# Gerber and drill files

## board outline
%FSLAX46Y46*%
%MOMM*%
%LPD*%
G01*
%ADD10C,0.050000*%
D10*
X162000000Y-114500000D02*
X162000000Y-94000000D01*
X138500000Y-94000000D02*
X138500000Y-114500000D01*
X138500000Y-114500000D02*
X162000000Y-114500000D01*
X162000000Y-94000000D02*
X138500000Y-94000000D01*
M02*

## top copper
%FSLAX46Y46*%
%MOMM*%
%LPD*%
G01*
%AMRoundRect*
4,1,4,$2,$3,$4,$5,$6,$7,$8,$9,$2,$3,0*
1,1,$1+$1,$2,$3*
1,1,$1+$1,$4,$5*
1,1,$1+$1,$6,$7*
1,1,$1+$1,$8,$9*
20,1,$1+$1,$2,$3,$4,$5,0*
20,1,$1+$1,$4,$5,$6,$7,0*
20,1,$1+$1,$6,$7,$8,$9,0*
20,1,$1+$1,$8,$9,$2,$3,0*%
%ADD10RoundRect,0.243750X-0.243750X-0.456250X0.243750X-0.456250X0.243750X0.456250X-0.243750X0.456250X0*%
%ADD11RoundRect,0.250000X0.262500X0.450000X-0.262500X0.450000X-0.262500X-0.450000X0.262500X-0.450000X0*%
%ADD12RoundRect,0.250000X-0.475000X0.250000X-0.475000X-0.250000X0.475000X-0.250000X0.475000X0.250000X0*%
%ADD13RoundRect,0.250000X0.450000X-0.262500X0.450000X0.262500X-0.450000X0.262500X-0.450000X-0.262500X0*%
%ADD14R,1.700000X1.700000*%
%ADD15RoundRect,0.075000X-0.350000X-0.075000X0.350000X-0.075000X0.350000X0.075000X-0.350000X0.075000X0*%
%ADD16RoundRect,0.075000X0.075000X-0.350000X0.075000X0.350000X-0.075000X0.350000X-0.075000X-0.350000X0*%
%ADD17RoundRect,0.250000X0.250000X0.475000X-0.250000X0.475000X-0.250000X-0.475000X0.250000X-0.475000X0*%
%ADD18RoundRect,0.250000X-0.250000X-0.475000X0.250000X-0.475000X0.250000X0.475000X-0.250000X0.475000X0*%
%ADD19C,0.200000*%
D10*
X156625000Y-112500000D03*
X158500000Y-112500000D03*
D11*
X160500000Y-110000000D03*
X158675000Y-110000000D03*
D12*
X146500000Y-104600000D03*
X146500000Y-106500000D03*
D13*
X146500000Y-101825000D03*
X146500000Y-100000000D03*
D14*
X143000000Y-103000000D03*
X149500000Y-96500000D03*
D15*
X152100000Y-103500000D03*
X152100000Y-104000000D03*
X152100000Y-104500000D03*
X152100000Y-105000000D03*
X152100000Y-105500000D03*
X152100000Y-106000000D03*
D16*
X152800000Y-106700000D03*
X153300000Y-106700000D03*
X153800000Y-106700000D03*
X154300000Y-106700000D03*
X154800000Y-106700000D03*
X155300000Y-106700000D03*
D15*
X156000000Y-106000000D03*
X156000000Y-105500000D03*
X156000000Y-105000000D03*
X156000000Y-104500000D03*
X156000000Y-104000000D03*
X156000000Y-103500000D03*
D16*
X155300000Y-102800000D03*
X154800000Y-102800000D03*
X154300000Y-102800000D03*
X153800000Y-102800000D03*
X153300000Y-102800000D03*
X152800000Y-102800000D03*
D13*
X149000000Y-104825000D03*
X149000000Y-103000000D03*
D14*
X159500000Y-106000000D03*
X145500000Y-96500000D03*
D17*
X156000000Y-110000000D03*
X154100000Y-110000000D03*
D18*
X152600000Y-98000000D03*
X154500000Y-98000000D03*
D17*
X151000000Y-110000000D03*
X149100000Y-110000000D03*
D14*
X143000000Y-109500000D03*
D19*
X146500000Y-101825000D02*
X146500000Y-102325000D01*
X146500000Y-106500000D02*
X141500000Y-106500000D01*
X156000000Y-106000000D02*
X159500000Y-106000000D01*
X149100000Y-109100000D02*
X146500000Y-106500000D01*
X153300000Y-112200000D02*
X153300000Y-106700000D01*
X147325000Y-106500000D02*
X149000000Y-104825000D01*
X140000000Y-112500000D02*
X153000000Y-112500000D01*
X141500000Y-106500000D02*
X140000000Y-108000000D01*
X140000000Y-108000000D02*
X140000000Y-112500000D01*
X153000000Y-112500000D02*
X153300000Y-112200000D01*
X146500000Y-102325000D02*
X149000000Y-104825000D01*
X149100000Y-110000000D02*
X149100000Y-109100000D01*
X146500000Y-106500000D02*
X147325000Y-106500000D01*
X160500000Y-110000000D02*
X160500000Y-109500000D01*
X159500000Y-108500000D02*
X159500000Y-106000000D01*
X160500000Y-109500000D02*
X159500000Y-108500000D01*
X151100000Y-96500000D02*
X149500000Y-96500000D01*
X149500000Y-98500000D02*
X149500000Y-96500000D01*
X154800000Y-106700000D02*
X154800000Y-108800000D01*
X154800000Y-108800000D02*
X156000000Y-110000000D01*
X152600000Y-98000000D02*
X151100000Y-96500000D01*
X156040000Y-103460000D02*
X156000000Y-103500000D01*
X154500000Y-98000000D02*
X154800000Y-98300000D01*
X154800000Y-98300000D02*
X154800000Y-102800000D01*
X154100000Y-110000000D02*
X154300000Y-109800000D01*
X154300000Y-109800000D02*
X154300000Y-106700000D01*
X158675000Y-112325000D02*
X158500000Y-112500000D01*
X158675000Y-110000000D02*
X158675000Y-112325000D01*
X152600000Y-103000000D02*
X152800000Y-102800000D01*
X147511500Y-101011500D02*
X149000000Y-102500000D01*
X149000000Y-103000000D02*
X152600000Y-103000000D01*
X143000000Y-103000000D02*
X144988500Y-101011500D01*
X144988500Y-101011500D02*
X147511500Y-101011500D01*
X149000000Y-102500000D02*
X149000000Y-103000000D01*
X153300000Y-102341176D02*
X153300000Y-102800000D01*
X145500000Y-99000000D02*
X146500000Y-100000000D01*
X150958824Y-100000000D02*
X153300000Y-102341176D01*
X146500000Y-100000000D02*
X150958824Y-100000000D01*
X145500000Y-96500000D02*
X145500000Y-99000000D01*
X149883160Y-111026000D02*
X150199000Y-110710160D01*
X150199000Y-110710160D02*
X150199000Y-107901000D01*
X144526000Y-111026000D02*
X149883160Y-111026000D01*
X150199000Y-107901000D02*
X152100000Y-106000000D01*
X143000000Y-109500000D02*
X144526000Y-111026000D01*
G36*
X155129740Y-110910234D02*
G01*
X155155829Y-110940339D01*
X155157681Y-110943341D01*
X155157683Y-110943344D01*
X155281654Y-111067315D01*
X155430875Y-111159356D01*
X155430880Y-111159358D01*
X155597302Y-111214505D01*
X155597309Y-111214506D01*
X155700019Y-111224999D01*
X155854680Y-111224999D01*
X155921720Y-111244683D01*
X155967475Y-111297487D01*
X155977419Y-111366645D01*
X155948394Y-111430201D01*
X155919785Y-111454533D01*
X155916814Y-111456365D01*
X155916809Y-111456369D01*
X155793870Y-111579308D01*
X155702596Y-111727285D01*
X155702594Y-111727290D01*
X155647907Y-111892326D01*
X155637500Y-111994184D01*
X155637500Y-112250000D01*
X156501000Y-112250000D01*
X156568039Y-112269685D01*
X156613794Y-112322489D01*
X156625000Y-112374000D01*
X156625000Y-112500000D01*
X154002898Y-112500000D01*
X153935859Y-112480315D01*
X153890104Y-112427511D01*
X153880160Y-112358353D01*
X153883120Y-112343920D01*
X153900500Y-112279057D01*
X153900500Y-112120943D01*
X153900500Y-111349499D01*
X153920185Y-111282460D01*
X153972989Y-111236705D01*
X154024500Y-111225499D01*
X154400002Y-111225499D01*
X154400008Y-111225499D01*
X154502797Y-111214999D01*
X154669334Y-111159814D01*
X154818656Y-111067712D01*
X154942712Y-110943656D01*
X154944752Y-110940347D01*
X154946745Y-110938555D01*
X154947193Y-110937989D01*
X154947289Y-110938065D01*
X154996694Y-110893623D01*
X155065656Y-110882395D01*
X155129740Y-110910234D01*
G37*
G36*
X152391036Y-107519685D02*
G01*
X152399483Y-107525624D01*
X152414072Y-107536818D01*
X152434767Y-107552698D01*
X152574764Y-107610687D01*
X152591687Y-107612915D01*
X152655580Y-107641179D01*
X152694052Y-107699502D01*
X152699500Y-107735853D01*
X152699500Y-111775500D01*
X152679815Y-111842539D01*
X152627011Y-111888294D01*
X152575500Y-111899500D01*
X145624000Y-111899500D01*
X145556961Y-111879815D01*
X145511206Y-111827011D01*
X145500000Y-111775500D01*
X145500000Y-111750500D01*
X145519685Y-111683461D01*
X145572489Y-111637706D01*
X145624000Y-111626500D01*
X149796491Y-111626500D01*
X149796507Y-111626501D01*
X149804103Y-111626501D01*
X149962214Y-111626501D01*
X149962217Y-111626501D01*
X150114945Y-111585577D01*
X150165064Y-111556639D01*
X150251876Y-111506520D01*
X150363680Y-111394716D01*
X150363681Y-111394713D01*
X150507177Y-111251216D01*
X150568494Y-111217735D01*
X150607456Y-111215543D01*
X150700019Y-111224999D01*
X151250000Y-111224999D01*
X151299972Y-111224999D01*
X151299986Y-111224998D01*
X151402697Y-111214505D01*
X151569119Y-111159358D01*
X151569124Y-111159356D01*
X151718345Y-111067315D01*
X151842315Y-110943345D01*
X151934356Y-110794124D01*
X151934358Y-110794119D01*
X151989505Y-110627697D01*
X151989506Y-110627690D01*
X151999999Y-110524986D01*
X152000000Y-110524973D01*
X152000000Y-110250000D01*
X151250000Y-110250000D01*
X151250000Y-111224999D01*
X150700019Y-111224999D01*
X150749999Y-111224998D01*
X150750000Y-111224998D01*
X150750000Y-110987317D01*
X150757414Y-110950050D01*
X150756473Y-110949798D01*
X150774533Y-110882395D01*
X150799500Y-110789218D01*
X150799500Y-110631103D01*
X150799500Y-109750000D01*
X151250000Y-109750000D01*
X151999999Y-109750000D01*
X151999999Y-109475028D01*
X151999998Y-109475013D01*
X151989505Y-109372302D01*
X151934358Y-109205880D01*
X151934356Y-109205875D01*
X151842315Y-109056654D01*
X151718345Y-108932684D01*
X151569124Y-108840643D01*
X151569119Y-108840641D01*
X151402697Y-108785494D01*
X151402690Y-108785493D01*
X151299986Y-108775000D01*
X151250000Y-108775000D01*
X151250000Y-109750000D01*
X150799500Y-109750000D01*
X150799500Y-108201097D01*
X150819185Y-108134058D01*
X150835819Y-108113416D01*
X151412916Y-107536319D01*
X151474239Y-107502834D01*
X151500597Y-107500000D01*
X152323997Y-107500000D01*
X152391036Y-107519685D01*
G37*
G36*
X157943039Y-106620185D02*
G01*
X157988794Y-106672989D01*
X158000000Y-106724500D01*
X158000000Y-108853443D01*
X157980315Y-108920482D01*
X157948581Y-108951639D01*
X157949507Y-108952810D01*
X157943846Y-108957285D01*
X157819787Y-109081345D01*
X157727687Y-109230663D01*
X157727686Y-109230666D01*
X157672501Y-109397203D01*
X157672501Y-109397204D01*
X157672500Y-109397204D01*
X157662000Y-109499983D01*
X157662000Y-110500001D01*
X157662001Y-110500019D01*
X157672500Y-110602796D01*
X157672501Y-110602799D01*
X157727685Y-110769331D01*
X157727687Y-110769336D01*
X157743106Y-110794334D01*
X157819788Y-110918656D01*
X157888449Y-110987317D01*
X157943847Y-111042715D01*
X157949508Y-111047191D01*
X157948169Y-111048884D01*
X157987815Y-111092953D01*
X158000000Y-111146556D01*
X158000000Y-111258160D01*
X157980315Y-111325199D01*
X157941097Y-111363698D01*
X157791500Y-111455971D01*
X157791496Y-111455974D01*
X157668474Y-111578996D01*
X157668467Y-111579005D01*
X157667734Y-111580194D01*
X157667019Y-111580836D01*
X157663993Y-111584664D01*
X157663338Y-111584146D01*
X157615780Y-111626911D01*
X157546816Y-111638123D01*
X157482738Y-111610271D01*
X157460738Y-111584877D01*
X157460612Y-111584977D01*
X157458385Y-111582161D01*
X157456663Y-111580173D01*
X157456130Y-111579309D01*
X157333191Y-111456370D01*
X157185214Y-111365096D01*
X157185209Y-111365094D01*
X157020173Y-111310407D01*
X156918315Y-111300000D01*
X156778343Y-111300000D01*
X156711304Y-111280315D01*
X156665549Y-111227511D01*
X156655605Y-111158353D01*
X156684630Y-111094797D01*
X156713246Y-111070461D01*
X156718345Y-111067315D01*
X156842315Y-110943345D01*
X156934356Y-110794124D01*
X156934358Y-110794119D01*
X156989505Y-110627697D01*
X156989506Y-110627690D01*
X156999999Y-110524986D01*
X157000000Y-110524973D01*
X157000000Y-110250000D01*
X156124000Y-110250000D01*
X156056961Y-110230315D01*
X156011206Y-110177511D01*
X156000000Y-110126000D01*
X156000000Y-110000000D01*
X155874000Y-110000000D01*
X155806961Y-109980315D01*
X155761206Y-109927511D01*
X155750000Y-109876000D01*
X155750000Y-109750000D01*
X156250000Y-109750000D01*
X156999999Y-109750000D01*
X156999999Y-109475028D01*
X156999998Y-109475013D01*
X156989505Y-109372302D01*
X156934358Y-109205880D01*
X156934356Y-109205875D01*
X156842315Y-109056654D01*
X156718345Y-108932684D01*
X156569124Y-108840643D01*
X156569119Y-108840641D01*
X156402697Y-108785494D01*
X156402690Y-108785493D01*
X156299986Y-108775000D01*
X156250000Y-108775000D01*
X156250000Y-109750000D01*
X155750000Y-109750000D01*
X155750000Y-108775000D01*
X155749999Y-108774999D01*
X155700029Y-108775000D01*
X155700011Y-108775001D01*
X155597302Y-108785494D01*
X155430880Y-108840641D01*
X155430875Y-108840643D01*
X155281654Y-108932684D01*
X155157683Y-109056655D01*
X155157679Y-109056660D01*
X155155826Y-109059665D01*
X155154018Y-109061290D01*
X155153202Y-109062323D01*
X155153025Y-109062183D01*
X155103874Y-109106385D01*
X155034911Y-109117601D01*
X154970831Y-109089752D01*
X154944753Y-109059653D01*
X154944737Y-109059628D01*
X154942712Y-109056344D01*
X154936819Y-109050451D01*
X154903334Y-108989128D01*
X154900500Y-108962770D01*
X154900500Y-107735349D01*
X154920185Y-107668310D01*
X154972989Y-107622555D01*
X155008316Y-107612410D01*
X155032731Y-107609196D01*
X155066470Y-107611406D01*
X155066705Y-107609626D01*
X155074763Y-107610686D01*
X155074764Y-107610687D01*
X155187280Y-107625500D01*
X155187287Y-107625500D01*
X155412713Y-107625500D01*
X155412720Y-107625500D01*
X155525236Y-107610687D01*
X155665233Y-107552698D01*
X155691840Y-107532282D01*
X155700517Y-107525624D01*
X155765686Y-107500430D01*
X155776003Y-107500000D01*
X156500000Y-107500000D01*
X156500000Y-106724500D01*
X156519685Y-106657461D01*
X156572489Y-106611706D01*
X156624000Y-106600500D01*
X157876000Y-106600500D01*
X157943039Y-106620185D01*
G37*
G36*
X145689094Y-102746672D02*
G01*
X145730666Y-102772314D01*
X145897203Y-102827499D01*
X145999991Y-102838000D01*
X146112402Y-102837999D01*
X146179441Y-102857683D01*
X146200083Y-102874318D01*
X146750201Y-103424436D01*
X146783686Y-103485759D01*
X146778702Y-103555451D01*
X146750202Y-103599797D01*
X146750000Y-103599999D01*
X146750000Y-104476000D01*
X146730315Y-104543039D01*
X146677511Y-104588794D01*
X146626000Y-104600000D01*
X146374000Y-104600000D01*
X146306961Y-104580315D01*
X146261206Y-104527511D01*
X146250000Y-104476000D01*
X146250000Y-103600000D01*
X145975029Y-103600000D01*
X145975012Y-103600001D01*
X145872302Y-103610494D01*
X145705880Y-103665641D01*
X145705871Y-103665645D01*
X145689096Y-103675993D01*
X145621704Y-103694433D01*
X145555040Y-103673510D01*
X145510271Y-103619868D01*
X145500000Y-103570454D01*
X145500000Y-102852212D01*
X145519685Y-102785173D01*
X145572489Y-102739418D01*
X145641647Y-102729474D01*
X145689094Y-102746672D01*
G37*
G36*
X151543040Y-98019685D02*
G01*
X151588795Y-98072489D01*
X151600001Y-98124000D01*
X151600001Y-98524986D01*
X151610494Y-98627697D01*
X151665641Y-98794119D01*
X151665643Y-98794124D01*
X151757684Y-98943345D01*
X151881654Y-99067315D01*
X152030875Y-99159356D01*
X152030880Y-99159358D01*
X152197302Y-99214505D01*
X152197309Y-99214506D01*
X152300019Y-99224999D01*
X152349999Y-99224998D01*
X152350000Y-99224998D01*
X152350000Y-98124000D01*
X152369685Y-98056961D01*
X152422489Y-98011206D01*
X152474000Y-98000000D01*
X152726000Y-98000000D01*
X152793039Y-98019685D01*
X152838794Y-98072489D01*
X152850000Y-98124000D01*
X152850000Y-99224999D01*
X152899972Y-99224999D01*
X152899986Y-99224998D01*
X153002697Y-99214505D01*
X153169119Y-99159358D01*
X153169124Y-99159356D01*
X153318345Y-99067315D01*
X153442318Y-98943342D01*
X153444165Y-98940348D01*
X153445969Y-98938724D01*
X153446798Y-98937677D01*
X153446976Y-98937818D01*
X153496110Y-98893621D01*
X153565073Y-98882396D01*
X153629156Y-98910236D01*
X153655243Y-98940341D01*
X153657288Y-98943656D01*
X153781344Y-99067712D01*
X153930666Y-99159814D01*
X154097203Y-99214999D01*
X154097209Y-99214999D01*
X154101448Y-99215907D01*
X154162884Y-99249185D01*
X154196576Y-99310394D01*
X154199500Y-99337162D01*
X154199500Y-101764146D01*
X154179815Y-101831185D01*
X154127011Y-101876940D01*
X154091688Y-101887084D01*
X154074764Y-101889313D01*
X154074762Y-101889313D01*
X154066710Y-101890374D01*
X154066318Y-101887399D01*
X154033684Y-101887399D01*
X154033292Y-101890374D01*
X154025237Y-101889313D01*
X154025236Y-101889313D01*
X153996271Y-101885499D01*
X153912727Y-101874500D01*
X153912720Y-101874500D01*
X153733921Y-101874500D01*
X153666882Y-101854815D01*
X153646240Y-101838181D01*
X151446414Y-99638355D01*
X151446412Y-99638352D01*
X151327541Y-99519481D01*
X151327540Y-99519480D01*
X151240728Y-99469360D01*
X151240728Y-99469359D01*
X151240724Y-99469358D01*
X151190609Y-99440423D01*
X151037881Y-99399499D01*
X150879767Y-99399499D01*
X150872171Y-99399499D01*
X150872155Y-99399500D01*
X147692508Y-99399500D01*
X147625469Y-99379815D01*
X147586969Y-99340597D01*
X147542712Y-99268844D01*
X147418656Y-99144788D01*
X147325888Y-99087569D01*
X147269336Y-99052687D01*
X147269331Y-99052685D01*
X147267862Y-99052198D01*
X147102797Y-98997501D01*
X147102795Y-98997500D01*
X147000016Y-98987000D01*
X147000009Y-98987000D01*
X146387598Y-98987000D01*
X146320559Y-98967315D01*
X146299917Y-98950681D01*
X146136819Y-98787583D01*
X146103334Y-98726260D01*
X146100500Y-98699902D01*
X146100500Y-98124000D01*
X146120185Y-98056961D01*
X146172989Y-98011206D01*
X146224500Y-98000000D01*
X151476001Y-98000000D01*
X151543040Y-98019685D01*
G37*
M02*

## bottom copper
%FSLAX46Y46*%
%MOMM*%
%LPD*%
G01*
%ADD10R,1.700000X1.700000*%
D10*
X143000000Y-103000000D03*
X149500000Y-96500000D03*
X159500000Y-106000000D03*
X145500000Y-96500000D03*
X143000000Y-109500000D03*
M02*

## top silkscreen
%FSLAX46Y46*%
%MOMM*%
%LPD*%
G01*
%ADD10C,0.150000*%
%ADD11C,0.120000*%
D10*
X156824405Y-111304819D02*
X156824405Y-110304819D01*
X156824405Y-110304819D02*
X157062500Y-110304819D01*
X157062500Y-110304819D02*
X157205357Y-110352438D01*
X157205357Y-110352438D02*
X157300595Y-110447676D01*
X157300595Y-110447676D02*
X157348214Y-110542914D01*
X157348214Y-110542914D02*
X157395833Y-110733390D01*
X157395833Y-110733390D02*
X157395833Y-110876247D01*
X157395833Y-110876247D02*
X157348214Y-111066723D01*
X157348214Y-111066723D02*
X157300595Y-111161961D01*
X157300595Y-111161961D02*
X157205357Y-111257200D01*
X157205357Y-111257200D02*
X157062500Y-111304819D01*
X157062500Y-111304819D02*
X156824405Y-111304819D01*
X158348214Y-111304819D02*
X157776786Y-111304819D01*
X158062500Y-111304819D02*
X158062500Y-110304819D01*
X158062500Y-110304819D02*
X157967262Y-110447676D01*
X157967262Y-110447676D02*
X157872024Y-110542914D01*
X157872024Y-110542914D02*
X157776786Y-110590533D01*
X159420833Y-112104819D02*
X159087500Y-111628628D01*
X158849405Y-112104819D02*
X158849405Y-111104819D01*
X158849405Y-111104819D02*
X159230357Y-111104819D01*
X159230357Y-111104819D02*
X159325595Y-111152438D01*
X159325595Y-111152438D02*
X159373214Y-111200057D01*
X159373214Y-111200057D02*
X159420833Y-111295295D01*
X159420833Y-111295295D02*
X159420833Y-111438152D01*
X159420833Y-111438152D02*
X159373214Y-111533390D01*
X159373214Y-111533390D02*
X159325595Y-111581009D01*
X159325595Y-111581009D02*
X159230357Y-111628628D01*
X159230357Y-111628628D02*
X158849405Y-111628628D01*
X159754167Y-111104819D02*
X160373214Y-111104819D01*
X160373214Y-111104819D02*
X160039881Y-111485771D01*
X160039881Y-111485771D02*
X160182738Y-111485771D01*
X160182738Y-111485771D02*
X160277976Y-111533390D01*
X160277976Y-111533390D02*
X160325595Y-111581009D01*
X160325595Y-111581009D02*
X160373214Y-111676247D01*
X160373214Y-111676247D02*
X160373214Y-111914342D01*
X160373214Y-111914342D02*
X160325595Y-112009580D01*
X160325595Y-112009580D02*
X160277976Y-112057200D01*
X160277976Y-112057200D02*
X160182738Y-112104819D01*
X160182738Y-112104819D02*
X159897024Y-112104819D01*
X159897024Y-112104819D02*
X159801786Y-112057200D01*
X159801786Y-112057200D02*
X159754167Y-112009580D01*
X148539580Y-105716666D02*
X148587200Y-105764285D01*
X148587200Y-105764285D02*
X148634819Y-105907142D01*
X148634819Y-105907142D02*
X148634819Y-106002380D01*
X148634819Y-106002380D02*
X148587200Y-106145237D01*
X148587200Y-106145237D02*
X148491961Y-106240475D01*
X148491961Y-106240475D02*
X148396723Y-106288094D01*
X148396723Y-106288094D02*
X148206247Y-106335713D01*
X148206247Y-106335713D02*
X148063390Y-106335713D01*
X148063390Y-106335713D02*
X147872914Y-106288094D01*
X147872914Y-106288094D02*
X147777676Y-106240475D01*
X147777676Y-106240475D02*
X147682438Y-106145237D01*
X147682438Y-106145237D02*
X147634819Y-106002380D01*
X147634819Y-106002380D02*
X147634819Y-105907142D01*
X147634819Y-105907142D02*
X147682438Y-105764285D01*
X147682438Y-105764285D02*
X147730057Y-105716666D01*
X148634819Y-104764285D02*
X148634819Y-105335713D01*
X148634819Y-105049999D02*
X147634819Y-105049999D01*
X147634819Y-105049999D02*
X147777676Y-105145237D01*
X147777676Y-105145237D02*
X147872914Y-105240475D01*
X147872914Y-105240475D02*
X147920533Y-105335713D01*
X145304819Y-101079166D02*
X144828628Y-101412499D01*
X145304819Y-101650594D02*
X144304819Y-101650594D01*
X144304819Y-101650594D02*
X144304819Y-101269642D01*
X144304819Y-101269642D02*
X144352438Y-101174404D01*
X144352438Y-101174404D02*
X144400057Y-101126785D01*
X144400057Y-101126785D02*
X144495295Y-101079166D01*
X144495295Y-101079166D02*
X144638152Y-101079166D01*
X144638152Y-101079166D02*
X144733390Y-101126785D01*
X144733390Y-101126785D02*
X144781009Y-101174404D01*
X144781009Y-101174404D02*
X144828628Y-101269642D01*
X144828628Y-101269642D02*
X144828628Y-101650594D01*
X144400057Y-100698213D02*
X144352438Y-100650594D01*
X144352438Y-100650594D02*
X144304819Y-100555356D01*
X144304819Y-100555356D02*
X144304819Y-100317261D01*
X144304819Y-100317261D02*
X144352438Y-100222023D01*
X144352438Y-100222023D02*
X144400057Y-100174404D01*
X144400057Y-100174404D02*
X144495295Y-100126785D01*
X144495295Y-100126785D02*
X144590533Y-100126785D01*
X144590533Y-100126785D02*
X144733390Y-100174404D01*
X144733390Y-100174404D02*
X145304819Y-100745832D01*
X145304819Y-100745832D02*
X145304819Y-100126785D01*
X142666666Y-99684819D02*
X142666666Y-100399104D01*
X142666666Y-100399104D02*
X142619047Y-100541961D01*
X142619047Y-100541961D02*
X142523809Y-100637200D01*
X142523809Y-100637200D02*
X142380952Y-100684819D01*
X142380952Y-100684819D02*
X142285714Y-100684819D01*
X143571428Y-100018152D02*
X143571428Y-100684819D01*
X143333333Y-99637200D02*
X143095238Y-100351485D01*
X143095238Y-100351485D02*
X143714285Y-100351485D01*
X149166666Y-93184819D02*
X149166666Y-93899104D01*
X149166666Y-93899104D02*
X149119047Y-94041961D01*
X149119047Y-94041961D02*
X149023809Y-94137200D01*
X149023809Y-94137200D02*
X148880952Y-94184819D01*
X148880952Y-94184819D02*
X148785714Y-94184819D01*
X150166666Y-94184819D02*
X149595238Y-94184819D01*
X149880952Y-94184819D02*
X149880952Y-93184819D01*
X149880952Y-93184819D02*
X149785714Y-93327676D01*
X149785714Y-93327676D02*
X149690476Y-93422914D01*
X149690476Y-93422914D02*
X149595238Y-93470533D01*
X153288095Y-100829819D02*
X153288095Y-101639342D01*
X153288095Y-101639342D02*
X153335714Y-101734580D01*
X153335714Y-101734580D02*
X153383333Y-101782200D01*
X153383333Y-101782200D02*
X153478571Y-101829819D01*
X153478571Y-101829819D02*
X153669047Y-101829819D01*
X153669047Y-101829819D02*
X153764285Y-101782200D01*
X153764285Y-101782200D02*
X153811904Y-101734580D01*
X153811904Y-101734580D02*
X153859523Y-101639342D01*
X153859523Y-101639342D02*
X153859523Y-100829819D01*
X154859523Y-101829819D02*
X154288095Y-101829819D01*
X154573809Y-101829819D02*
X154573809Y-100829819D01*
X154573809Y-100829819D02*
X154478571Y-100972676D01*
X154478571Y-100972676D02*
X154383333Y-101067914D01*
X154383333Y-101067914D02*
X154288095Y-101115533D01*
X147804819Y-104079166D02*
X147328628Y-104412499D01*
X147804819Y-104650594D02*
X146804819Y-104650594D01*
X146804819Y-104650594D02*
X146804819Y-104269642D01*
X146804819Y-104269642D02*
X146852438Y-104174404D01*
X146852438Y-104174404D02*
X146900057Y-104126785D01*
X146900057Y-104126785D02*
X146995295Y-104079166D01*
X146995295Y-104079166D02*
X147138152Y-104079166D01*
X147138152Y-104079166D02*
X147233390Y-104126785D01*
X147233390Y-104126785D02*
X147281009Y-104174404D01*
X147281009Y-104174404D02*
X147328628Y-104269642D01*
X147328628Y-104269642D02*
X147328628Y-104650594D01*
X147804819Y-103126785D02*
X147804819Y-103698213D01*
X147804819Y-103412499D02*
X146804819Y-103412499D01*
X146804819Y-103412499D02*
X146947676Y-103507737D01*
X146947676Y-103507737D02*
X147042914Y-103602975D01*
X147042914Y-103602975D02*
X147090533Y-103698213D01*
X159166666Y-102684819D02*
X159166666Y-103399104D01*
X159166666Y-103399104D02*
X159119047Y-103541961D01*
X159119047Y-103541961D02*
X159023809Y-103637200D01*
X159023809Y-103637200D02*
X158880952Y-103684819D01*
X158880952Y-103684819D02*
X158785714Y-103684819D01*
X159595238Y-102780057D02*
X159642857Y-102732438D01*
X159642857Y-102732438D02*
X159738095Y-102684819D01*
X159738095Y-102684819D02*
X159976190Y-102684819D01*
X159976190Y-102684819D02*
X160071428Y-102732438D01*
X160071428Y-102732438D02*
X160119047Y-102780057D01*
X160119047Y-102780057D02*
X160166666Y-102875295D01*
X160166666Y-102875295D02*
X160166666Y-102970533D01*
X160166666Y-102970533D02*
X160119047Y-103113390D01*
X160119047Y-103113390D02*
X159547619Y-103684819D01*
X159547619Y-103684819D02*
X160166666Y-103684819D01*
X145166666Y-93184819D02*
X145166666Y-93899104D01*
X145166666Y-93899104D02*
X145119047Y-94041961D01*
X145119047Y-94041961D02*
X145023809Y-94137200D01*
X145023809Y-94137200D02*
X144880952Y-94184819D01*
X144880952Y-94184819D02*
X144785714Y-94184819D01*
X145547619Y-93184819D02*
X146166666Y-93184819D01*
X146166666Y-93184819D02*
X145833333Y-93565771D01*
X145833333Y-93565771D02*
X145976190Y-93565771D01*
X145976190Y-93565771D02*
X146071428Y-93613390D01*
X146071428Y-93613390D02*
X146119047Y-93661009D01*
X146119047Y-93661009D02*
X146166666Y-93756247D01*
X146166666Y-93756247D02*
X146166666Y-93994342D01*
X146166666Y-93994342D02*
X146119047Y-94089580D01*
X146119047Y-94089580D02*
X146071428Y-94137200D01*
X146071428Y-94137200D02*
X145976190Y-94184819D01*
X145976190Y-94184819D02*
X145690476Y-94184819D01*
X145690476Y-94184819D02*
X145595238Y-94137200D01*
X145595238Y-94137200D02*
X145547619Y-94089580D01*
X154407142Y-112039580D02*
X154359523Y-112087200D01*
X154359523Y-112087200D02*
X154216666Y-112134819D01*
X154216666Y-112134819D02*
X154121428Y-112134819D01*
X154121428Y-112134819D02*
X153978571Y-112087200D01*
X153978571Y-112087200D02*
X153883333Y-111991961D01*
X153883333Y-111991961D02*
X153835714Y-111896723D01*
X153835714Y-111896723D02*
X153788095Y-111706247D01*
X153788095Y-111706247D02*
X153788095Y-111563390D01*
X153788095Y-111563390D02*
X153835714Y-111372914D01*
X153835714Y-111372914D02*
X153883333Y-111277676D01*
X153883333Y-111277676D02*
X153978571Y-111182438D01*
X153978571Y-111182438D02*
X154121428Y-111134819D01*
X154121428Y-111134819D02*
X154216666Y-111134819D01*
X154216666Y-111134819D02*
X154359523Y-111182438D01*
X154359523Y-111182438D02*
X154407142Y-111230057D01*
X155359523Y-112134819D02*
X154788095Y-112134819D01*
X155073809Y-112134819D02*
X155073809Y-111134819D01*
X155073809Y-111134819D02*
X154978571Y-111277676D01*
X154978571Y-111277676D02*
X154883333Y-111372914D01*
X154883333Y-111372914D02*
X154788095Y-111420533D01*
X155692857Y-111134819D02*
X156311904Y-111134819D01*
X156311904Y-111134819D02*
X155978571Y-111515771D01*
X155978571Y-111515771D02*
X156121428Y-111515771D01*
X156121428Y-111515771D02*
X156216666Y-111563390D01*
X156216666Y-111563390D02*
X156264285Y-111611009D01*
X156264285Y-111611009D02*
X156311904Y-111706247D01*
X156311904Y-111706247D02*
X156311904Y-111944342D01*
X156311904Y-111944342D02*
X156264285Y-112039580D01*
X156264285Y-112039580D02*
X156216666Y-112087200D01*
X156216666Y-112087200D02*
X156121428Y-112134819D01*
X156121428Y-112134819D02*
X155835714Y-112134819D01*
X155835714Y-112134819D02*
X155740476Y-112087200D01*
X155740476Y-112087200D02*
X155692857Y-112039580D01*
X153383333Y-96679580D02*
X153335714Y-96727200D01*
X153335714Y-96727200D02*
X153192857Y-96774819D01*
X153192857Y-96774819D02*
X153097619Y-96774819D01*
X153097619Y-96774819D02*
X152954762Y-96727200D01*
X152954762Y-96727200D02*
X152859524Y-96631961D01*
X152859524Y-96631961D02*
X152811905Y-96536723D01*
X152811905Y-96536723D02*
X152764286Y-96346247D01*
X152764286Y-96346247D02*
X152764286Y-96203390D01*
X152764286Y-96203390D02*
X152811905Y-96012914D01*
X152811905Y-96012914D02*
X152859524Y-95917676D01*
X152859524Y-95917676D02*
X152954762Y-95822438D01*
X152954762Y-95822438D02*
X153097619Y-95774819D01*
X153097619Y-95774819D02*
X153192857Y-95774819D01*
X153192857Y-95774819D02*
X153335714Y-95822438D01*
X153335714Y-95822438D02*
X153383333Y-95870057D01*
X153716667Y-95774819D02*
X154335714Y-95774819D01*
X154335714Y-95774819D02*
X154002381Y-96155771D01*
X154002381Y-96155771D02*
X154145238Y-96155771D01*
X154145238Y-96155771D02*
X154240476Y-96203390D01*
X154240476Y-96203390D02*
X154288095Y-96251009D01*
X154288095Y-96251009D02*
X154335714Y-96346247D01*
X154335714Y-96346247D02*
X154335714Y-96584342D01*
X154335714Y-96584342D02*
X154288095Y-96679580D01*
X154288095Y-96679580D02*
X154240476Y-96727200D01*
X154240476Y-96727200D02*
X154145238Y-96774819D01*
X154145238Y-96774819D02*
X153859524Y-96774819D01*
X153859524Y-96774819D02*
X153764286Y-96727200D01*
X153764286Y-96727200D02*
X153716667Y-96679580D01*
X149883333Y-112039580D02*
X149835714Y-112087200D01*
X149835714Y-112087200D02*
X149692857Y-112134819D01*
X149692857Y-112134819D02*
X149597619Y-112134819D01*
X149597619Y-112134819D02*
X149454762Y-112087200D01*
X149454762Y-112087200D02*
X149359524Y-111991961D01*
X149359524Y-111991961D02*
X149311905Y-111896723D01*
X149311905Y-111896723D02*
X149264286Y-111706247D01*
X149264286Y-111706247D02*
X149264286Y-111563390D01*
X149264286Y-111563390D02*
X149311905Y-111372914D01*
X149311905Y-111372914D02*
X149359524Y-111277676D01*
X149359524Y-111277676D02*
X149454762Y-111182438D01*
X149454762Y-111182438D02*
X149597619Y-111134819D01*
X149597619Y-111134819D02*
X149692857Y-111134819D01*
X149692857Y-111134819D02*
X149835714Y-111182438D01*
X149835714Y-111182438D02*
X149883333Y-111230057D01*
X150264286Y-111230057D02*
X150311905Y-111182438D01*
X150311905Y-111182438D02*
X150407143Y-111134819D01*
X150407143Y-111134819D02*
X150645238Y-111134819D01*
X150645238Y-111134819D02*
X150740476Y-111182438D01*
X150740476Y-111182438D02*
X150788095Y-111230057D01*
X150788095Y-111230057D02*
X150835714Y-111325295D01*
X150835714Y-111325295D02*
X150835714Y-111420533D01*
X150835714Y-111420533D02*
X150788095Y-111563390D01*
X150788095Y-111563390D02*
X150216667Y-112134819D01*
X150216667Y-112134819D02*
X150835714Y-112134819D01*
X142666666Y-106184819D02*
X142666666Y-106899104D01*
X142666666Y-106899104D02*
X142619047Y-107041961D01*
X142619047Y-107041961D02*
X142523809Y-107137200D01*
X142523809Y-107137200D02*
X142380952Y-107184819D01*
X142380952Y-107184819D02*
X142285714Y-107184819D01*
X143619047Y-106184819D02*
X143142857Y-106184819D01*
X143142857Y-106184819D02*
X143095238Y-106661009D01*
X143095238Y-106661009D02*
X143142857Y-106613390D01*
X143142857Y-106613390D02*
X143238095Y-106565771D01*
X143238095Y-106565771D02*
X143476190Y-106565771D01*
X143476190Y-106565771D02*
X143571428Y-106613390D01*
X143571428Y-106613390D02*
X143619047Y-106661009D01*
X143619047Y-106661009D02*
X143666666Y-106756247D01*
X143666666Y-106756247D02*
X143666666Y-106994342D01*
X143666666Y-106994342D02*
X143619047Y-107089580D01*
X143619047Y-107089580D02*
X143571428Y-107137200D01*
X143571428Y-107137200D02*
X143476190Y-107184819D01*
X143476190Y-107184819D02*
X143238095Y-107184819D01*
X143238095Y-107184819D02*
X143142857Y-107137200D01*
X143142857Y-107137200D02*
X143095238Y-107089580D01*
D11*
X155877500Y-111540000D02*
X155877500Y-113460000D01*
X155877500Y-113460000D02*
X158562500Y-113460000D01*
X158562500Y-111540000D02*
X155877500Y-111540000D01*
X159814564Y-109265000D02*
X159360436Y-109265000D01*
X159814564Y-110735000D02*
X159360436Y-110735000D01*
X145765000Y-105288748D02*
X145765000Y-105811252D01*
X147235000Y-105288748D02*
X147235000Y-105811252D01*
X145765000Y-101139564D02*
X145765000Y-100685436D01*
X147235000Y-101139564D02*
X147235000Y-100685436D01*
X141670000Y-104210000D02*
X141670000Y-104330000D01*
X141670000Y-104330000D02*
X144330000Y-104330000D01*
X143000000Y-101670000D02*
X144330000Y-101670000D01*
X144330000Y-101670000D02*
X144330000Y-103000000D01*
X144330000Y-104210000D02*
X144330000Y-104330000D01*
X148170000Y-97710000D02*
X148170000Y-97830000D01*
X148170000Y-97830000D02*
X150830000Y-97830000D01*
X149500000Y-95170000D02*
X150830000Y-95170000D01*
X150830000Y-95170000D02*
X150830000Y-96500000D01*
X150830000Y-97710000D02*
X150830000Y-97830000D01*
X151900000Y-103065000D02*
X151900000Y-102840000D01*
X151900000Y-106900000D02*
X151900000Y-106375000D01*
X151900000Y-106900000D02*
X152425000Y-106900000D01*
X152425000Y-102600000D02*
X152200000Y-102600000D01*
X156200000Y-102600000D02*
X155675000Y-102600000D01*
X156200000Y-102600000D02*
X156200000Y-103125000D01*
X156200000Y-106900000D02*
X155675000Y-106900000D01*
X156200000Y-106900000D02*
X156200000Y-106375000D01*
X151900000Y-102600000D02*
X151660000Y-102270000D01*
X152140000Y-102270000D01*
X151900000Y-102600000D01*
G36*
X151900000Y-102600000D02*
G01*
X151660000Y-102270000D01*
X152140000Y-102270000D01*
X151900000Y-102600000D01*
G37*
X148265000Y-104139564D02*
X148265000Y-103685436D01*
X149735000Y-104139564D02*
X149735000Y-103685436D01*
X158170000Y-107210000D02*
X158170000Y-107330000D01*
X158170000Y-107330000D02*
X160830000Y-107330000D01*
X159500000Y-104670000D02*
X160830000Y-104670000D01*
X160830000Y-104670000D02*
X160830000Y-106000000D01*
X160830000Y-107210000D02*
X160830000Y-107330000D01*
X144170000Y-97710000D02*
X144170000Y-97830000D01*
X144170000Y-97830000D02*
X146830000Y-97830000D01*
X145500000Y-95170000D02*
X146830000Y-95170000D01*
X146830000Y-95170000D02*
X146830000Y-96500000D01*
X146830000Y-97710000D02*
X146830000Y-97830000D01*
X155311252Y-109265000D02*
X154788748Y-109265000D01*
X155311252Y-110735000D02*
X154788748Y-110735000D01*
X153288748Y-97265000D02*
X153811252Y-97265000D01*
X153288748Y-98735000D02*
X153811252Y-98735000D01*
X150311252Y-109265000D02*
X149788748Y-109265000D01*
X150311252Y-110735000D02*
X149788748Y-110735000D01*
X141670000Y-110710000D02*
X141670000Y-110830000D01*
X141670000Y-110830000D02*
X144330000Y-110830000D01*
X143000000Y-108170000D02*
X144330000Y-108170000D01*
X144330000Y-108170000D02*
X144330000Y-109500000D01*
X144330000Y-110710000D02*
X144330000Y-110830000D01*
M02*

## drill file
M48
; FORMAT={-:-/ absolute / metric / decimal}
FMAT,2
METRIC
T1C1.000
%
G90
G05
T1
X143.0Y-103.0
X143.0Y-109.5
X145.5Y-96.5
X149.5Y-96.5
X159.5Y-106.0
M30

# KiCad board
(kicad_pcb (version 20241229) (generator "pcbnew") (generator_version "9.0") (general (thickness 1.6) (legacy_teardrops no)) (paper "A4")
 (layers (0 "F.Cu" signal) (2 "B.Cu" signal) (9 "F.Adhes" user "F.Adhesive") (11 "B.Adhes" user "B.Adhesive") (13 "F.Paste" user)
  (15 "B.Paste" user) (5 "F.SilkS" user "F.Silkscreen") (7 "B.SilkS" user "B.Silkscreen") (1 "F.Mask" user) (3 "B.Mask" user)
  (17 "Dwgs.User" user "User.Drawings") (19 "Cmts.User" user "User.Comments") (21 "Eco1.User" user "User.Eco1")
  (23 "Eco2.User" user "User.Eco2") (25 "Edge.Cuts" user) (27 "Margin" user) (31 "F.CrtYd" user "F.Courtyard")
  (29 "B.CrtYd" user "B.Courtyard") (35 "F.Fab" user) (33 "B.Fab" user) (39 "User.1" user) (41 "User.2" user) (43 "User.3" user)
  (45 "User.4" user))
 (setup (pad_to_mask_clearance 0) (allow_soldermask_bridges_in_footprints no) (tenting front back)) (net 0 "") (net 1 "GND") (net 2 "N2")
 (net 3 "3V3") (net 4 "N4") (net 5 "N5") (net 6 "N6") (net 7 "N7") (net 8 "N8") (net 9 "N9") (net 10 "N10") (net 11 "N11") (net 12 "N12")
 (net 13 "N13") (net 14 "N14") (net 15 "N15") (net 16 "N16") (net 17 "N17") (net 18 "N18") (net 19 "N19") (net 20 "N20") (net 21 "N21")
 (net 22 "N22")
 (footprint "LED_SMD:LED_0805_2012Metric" (layer "F.Cu") (at 157.5625 112.5)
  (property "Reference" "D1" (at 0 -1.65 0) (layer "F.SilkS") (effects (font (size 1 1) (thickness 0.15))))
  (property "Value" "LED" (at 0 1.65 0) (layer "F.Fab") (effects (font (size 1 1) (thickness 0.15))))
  (fp_line (start -1.685 -0.96) (end -1.685 0.96) (stroke (width 0.12) (type solid)) (layer "F.SilkS"))
  (fp_line (start -1.685 0.96) (end 1 0.96) (stroke (width 0.12) (type solid)) (layer "F.SilkS"))
  (fp_line (start 1 -0.96) (end -1.685 -0.96) (stroke (width 0.12) (type solid)) (layer "F.SilkS"))
  (pad "1" smd roundrect (at -0.9375 0) (size 0.975 1.4) (layers "F.Cu" "F.Mask" "F.Paste") (roundrect_rratio 0.25) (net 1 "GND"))
  (pad "2" smd roundrect (at 0.9375 0) (size 0.975 1.4) (layers "F.Cu" "F.Mask" "F.Paste") (roundrect_rratio 0.25) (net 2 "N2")))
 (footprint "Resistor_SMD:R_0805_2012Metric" (layer "F.Cu") (at 159.5875 110 180)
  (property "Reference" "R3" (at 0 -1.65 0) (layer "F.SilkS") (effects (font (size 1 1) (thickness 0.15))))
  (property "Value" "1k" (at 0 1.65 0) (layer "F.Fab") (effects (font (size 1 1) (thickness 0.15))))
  (fp_line (start -0.227064 0.735) (end 0.227064 0.735) (stroke (width 0.12) (type solid)) (layer "F.SilkS"))
  (fp_line (start -0.227064 -0.735) (end 0.227064 -0.735) (stroke (width 0.12) (type solid)) (layer "F.SilkS"))
  (pad "1" smd roundrect (at -0.9125 0 180) (size 1.025 1.4) (layers "F.Cu" "F.Mask" "F.Paste") (roundrect_rratio 0.243902) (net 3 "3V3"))
  (pad "2" smd roundrect (at 0.9125 0 180) (size 1.025 1.4) (layers "F.Cu" "F.Mask" "F.Paste") (roundrect_rratio 0.243902) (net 2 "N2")))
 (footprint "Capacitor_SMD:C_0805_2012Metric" (layer "F.Cu") (at 146.5 105.55 -90)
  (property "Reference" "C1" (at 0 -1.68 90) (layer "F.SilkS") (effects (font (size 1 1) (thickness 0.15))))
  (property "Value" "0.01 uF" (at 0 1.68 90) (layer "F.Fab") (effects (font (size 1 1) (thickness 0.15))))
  (fp_line (start -0.261252 0.735) (end 0.261252 0.735) (stroke (width 0.12) (type solid)) (layer "F.SilkS"))
  (fp_line (start -0.261252 -0.735) (end 0.261252 -0.735) (stroke (width 0.12) (type solid)) (layer "F.SilkS"))
  (pad "1" smd roundrect (at -0.95 0 270) (size 1 1.45) (layers "F.Cu" "F.Mask" "F.Paste") (roundrect_rratio 0.25) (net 1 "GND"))
  (pad "2" smd roundrect (at 0.95 0 270) (size 1 1.45) (layers "F.Cu" "F.Mask" "F.Paste") (roundrect_rratio 0.25) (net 3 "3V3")))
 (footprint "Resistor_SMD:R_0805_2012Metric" (layer "F.Cu") (at 146.5 100.9125 90)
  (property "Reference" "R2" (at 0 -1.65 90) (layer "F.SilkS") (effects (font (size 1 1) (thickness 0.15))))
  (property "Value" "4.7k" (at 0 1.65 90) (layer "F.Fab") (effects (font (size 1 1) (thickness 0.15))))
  (fp_line (start -0.227064 -0.735) (end 0.227064 -0.735) (stroke (width 0.12) (type solid)) (layer "F.SilkS"))
  (fp_line (start -0.227064 0.735) (end 0.227064 0.735) (stroke (width 0.12) (type solid)) (layer "F.SilkS"))
  (pad "1" smd roundrect (at -0.9125 0 90) (size 1.025 1.4) (layers "F.Cu" "F.Mask" "F.Paste") (roundrect_rratio 0.243902) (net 3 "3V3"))
  (pad "2" smd roundrect (at 0.9125 0 90) (size 1.025 1.4) (layers "F.Cu" "F.Mask" "F.Paste") (roundrect_rratio 0.243902) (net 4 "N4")))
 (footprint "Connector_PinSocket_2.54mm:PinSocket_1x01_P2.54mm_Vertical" (layer "F.Cu") (at 143 103)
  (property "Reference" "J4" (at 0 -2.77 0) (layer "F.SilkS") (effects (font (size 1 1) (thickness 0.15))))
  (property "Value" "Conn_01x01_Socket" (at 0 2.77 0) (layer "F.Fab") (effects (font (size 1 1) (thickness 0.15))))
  (fp_line (start -1.33 1.21) (end -1.33 1.33) (stroke (width 0.12) (type solid)) (layer "F.SilkS"))
  (fp_line (start -1.33 1.33) (end 1.33 1.33) (stroke (width 0.12) (type solid)) (layer "F.SilkS"))
  (fp_line (start 0 -1.33) (end 1.33 -1.33) (stroke (width 0.12) (type solid)) (layer "F.SilkS"))
  (fp_line (start 1.33 -1.33) (end 1.33 0) (stroke (width 0.12) (type solid)) (layer "F.SilkS"))
  (fp_line (start 1.33 1.21) (end 1.33 1.33) (stroke (width 0.12) (type solid)) (layer "F.SilkS"))
  (pad "1" thru_hole rect (at 0 0) (size 1.7 1.7) (drill 1) (layers "*.Cu" "*.Mask") (remove_unused_layers no) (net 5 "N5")))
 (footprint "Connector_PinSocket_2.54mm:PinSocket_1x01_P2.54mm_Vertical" (layer "F.Cu") (at 149.5 96.5)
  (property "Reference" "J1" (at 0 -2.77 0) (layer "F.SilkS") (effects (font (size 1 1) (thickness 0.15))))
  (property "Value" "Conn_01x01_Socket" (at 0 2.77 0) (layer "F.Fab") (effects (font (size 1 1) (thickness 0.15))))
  (fp_line (start -1.33 1.21) (end -1.33 1.33) (stroke (width 0.12) (type solid)) (layer "F.SilkS"))
  (fp_line (start -1.33 1.33) (end 1.33 1.33) (stroke (width 0.12) (type solid)) (layer "F.SilkS"))
  (fp_line (start 0 -1.33) (end 1.33 -1.33) (stroke (width 0.12) (type solid)) (layer "F.SilkS"))
  (fp_line (start 1.33 -1.33) (end 1.33 0) (stroke (width 0.12) (type solid)) (layer "F.SilkS"))
  (fp_line (start 1.33 1.21) (end 1.33 1.33) (stroke (width 0.12) (type solid)) (layer "F.SilkS"))
  (pad "1" thru_hole rect (at 0 0) (size 1.7 1.7) (drill 1) (layers "*.Cu" "*.Mask") (remove_unused_layers no) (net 1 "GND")))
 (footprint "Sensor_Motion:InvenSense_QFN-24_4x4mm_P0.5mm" (layer "F.Cu") (at 154.05 104.75)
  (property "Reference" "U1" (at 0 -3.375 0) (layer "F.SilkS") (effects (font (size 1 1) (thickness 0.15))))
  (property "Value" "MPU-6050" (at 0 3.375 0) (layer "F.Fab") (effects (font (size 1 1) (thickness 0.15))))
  (fp_line (start -2.15 -1.685) (end -2.15 -1.91) (stroke (width 0.12) (type solid)) (layer "F.SilkS"))
  (fp_line (start -2.15 2.15) (end -2.15 1.625) (stroke (width 0.12) (type solid)) (layer "F.SilkS"))
  (fp_line (start -2.15 2.15) (end -1.625 2.15) (stroke (width 0.12) (type solid)) (layer "F.SilkS"))
  (fp_line (start -1.625 -2.15) (end -1.85 -2.15) (stroke (width 0.12) (type solid)) (layer "F.SilkS"))
  (fp_line (start 2.15 -2.15) (end 1.625 -2.15) (stroke (width 0.12) (type solid)) (layer "F.SilkS"))
  (fp_line (start 2.15 -2.15) (end 2.15 -1.625) (stroke (width 0.12) (type solid)) (layer "F.SilkS"))
  (fp_line (start 2.15 2.15) (end 1.625 2.15) (stroke (width 0.12) (type solid)) (layer "F.SilkS"))
  (fp_line (start 2.15 2.15) (end 2.15 1.625) (stroke (width 0.12) (type solid)) (layer "F.SilkS"))
  (fp_poly
   (pts (xy -2.15 -2.15) (xy -2.39 -2.48) (xy -1.91 -2.48) (xy -2.15 -2.15)) (stroke (width 0.12) (type solid)) (fill yes) (layer "F.SilkS"))
  (pad "1" smd roundrect (at -1.95 -1.25) (size 0.85 0.3) (layers "F.Cu" "F.Mask" "F.Paste") (roundrect_rratio 0.25) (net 1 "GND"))
  (pad "2" smd roundrect (at -1.95 -0.75) (size 0.85 0.3) (layers "F.Cu" "F.Mask" "F.Paste") (roundrect_rratio 0.25) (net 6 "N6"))
  (pad "3" smd roundrect (at -1.95 -0.25) (size 0.85 0.3) (layers "F.Cu" "F.Mask" "F.Paste") (roundrect_rratio 0.25) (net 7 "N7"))
  (pad "4" smd roundrect (at -1.95 0.25) (size 0.85 0.3) (layers "F.Cu" "F.Mask" "F.Paste") (roundrect_rratio 0.25) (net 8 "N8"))
  (pad "5" smd roundrect (at -1.95 0.75) (size 0.85 0.3) (layers "F.Cu" "F.Mask" "F.Paste") (roundrect_rratio 0.25) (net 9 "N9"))
  (pad "6" smd roundrect (at -1.95 1.25) (size 0.85 0.3) (layers "F.Cu" "F.Mask" "F.Paste") (roundrect_rratio 0.25) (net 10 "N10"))
  (pad "7" smd roundrect (at -1.25 1.95 90) (size 0.85 0.3) (layers "F.Cu" "F.Mask" "F.Paste") (roundrect_rratio 0.25) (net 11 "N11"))
  (pad "8" smd roundrect (at -0.75 1.95 90) (size 0.85 0.3) (layers "F.Cu" "F.Mask" "F.Paste") (roundrect_rratio 0.25) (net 3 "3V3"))
  (pad "9" smd roundrect (at -0.25 1.95 90) (size 0.85 0.3) (layers "F.Cu" "F.Mask" "F.Paste") (roundrect_rratio 0.25) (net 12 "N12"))
  (pad "10" smd roundrect (at 0.25 1.95 90) (size 0.85 0.3) (layers "F.Cu" "F.Mask" "F.Paste") (roundrect_rratio 0.25) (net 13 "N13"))
  (pad "11" smd roundrect (at 0.75 1.95 90) (size 0.85 0.3) (layers "F.Cu" "F.Mask" "F.Paste") (roundrect_rratio 0.25) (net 1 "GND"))
  (pad "12" smd roundrect (at 1.25 1.95 90) (size 0.85 0.3) (layers "F.Cu" "F.Mask" "F.Paste") (roundrect_rratio 0.25) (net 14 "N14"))
  (pad "13" smd roundrect (at 1.95 1.25) (size 0.85 0.3) (layers "F.Cu" "F.Mask" "F.Paste") (roundrect_rratio 0.25) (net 3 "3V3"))
  (pad "14" smd roundrect (at 1.95 0.75) (size 0.85 0.3) (layers "F.Cu" "F.Mask" "F.Paste") (roundrect_rratio 0.25) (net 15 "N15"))
  (pad "15" smd roundrect (at 1.95 0.25) (size 0.85 0.3) (layers "F.Cu" "F.Mask" "F.Paste") (roundrect_rratio 0.25) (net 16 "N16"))
  (pad "16" smd roundrect (at 1.95 -0.25) (size 0.85 0.3) (layers "F.Cu" "F.Mask" "F.Paste") (roundrect_rratio 0.25) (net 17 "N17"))
  (pad "17" smd roundrect (at 1.95 -0.75) (size 0.85 0.3) (layers "F.Cu" "F.Mask" "F.Paste") (roundrect_rratio 0.25) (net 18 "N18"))
  (pad "18" smd roundrect (at 1.95 -1.25) (size 0.85 0.3) (layers "F.Cu" "F.Mask" "F.Paste") (roundrect_rratio 0.25) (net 1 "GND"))
  (pad "19" smd roundrect (at 1.25 -1.95 90) (size 0.85 0.3) (layers "F.Cu" "F.Mask" "F.Paste") (roundrect_rratio 0.25) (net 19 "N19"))
  (pad "20" smd roundrect (at 0.75 -1.95 90) (size 0.85 0.3) (layers "F.Cu" "F.Mask" "F.Paste") (roundrect_rratio 0.25) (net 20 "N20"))
  (pad "21" smd roundrect (at 0.25 -1.95 90) (size 0.85 0.3) (layers "F.Cu" "F.Mask" "F.Paste") (roundrect_rratio 0.25) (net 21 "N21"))
  (pad "22" smd roundrect (at -0.25 -1.95 90) (size 0.85 0.3) (layers "F.Cu" "F.Mask" "F.Paste") (roundrect_rratio 0.25) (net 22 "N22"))
  (pad "23" smd roundrect (at -0.75 -1.95 90) (size 0.85 0.3) (layers "F.Cu" "F.Mask" "F.Paste") (roundrect_rratio 0.25) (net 4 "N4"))
  (pad "24" smd roundrect (at -1.25 -1.95 90) (size 0.85 0.3) (layers "F.Cu" "F.Mask" "F.Paste") (roundrect_rratio 0.25) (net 5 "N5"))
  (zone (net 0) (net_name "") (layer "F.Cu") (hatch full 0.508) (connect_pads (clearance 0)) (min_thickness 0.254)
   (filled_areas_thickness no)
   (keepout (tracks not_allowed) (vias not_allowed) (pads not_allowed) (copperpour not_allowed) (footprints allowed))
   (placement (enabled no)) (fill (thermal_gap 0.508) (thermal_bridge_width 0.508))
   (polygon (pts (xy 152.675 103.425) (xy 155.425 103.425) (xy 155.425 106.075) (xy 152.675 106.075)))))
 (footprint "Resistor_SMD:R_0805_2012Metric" (layer "F.Cu") (at 149 103.9125 90)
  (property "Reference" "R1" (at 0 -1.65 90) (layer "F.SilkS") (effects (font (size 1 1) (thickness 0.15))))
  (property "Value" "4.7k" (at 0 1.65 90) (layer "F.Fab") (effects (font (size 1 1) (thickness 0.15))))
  (fp_line (start -0.227064 -0.735) (end 0.227064 -0.735) (stroke (width 0.12) (type solid)) (layer "F.SilkS"))
  (fp_line (start -0.227064 0.735) (end 0.227064 0.735) (stroke (width 0.12) (type solid)) (layer "F.SilkS"))
  (pad "1" smd roundrect (at -0.9125 0 90) (size 1.025 1.4) (layers "F.Cu" "F.Mask" "F.Paste") (roundrect_rratio 0.243902) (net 3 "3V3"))
  (pad "2" smd roundrect (at 0.9125 0 90) (size 1.025 1.4) (layers "F.Cu" "F.Mask" "F.Paste") (roundrect_rratio 0.243902) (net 5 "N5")))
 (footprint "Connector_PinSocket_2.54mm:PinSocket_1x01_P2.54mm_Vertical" (layer "F.Cu") (at 159.5 106)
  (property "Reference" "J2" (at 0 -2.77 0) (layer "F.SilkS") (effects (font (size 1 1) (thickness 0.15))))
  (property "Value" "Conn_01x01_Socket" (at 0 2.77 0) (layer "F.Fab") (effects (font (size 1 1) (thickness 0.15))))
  (fp_line (start -1.33 1.21) (end -1.33 1.33) (stroke (width 0.12) (type solid)) (layer "F.SilkS"))
  (fp_line (start -1.33 1.33) (end 1.33 1.33) (stroke (width 0.12) (type solid)) (layer "F.SilkS"))
  (fp_line (start 0 -1.33) (end 1.33 -1.33) (stroke (width 0.12) (type solid)) (layer "F.SilkS"))
  (fp_line (start 1.33 -1.33) (end 1.33 0) (stroke (width 0.12) (type solid)) (layer "F.SilkS"))
  (fp_line (start 1.33 1.21) (end 1.33 1.33) (stroke (width 0.12) (type solid)) (layer "F.SilkS"))
  (pad "1" thru_hole rect (at 0 0) (size 1.7 1.7) (drill 1) (layers "*.Cu" "*.Mask") (remove_unused_layers no) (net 3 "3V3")))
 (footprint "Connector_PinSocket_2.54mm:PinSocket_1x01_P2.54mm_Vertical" (layer "F.Cu") (at 145.5 96.5)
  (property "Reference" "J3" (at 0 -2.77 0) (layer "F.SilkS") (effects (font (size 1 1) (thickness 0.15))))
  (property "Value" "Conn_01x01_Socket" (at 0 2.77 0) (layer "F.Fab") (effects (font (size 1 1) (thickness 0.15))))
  (fp_line (start -1.33 1.21) (end -1.33 1.33) (stroke (width 0.12) (type solid)) (layer "F.SilkS"))
  (fp_line (start -1.33 1.33) (end 1.33 1.33) (stroke (width 0.12) (type solid)) (layer "F.SilkS"))
  (fp_line (start 0 -1.33) (end 1.33 -1.33) (stroke (width 0.12) (type solid)) (layer "F.SilkS"))
  (fp_line (start 1.33 -1.33) (end 1.33 0) (stroke (width 0.12) (type solid)) (layer "F.SilkS"))
  (fp_line (start 1.33 1.21) (end 1.33 1.33) (stroke (width 0.12) (type solid)) (layer "F.SilkS"))
  (pad "1" thru_hole rect (at 0 0) (size 1.7 1.7) (drill 1) (layers "*.Cu" "*.Mask") (remove_unused_layers no) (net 4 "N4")))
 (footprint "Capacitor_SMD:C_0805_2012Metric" (layer "F.Cu") (at 155.05 110 180)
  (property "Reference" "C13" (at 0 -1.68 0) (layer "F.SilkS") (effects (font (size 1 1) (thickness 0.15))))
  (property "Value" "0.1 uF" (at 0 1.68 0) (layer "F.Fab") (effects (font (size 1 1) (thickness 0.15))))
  (fp_line (start -0.261252 0.735) (end 0.261252 0.735) (stroke (width 0.12) (type solid)) (layer "F.SilkS"))
  (fp_line (start -0.261252 -0.735) (end 0.261252 -0.735) (stroke (width 0.12) (type solid)) (layer "F.SilkS"))
  (pad "1" smd roundrect (at -0.95 0 180) (size 1 1.45) (layers "F.Cu" "F.Mask" "F.Paste") (roundrect_rratio 0.25) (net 1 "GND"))
  (pad "2" smd roundrect (at 0.95 0 180) (size 1 1.45) (layers "F.Cu" "F.Mask" "F.Paste") (roundrect_rratio 0.25) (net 13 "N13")))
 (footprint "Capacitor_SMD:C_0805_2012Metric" (layer "F.Cu") (at 153.55 98)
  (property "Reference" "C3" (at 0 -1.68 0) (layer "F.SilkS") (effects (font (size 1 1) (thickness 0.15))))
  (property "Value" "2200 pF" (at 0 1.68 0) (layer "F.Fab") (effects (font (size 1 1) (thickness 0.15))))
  (fp_line (start -0.261252 -0.735) (end 0.261252 -0.735) (stroke (width 0.12) (type solid)) (layer "F.SilkS"))
  (fp_line (start -0.261252 0.735) (end 0.261252 0.735) (stroke (width 0.12) (type solid)) (layer "F.SilkS"))
  (pad "1" smd roundrect (at -0.95 0) (size 1 1.45) (layers "F.Cu" "F.Mask" "F.Paste") (roundrect_rratio 0.25) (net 1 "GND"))
  (pad "2" smd roundrect (at 0.95 0) (size 1 1.45) (layers "F.Cu" "F.Mask" "F.Paste") (roundrect_rratio 0.25) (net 20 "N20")))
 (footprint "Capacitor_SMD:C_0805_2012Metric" (layer "F.Cu") (at 150.05 110 180)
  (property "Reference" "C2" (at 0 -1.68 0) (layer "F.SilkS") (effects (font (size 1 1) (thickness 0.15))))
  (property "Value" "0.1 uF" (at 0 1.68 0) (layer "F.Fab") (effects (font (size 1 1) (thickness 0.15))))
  (fp_line (start -0.261252 0.735) (end 0.261252 0.735) (stroke (width 0.12) (type solid)) (layer "F.SilkS"))
  (fp_line (start -0.261252 -0.735) (end 0.261252 -0.735) (stroke (width 0.12) (type solid)) (layer "F.SilkS"))
  (pad "1" smd roundrect (at -0.95 0 180) (size 1 1.45) (layers "F.Cu" "F.Mask" "F.Paste") (roundrect_rratio 0.25) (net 1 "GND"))
  (pad "2" smd roundrect (at 0.95 0 180) (size 1 1.45) (layers "F.Cu" "F.Mask" "F.Paste") (roundrect_rratio 0.25) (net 3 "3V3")))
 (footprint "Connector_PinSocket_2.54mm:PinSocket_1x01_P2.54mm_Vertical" (layer "F.Cu") (at 143 109.5)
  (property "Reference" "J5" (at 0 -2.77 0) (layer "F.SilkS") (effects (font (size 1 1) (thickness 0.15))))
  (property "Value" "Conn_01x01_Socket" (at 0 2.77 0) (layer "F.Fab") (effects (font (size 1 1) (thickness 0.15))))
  (fp_line (start -1.33 1.21) (end -1.33 1.33) (stroke (width 0.12) (type solid)) (layer "F.SilkS"))
  (fp_line (start -1.33 1.33) (end 1.33 1.33) (stroke (width 0.12) (type solid)) (layer "F.SilkS"))
  (fp_line (start 0 -1.33) (end 1.33 -1.33) (stroke (width 0.12) (type solid)) (layer "F.SilkS"))
  (fp_line (start 1.33 -1.33) (end 1.33 0) (stroke (width 0.12) (type solid)) (layer "F.SilkS"))
  (fp_line (start 1.33 1.21) (end 1.33 1.33) (stroke (width 0.12) (type solid)) (layer "F.SilkS"))
  (pad "1" thru_hole rect (at 0 0) (size 1.7 1.7) (drill 1) (layers "*.Cu" "*.Mask") (remove_unused_layers no) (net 10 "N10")))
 (gr_line (start 162 114.5) (end 162 94) (stroke (width 0.05) (type default)) (layer "Edge.Cuts"))
 (gr_line (start 138.5 94) (end 138.5 114.5) (stroke (width 0.05) (type default)) (layer "Edge.Cuts"))
 (gr_line (start 138.5 114.5) (end 162 114.5) (stroke (width 0.05) (type default)) (layer "Edge.Cuts"))
 (gr_line (start 162 94) (end 138.5 94) (stroke (width 0.05) (type default)) (layer "Edge.Cuts"))
 (segment (start 146.5 101.825) (end 146.5 102.325) (width 0.2) (layer "F.Cu") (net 3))
 (segment (start 146.5 106.5) (end 141.5 106.5) (width 0.2) (layer "F.Cu") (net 3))
 (segment (start 156 106) (end 159.5 106) (width 0.2) (layer "F.Cu") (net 3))
 (segment (start 149.1 109.1) (end 146.5 106.5) (width 0.2) (layer "F.Cu") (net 3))
 (segment (start 153.3 112.2) (end 153.3 106.7) (width 0.2) (layer "F.Cu") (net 3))
 (segment (start 147.325 106.5) (end 149 104.825) (width 0.2) (layer "F.Cu") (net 3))
 (segment (start 140 112.5) (end 153 112.5) (width 0.2) (layer "F.Cu") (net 3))
 (segment (start 141.5 106.5) (end 140 108) (width 0.2) (layer "F.Cu") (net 3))
 (segment (start 140 108) (end 140 112.5) (width 0.2) (layer "F.Cu") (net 3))
 (segment (start 153 112.5) (end 153.3 112.2) (width 0.2) (layer "F.Cu") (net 3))
 (segment (start 146.5 102.325) (end 149 104.825) (width 0.2) (layer "F.Cu") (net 3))
 (segment (start 149.1 110) (end 149.1 109.1) (width 0.2) (layer "F.Cu") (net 3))
 (segment (start 146.5 106.5) (end 147.325 106.5) (width 0.2) (layer "F.Cu") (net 3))
 (segment (start 160.5 110) (end 160.5 109.5) (width 0.2) (layer "F.Cu") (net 3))
 (segment (start 159.5 108.5) (end 159.5 106) (width 0.2) (layer "F.Cu") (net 3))
 (segment (start 160.5 109.5) (end 159.5 108.5) (width 0.2) (layer "F.Cu") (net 3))
 (segment (start 151.1 96.5) (end 149.5 96.5) (width 0.2) (layer "F.Cu") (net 1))
 (segment (start 149.5 98.5) (end 149.5 96.5) (width 0.2) (layer "F.Cu") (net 1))
 (segment (start 154.8 106.7) (end 154.8 108.8) (width 0.2) (layer "F.Cu") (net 1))
 (segment (start 154.8 108.8) (end 156 110) (width 0.2) (layer "F.Cu") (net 1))
 (segment (start 152.6 98) (end 151.1 96.5) (width 0.2) (layer "F.Cu") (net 1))
 (segment (start 156.04 103.46) (end 156 103.5) (width 0.2) (layer "F.Cu") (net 1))
 (segment (start 154.5 98) (end 154.8 98.3) (width 0.2) (layer "F.Cu") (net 20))
 (segment (start 154.8 98.3) (end 154.8 102.8) (width 0.2) (layer "F.Cu") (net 20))
 (segment (start 154.1 110) (end 154.3 109.8) (width 0.2) (layer "F.Cu") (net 13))
 (segment (start 154.3 109.8) (end 154.3 106.7) (width 0.2) (layer "F.Cu") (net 13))
 (segment (start 158.675 112.325) (end 158.5 112.5) (width 0.2) (layer "F.Cu") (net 2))
 (segment (start 158.675 110) (end 158.675 112.325) (width 0.2) (layer "F.Cu") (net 2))
 (segment (start 152.6 103) (end 152.8 102.8) (width 0.2) (layer "F.Cu") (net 5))
 (segment (start 147.5115 101.0115) (end 149 102.5) (width 0.2) (layer "F.Cu") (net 5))
 (segment (start 149 103) (end 152.6 103) (width 0.2) (layer "F.Cu") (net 5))
 (segment (start 143 103) (end 144.9885 101.0115) (width 0.2) (layer "F.Cu") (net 5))
 (segment (start 144.9885 101.0115) (end 147.5115 101.0115) (width 0.2) (layer "F.Cu") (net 5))
 (segment (start 149 102.5) (end 149 103) (width 0.2) (layer "F.Cu") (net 5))
 (segment (start 153.3 102.341176) (end 153.3 102.8) (width 0.2) (layer "F.Cu") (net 4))
 (segment (start 145.5 99) (end 146.5 100) (width 0.2) (layer "F.Cu") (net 4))
 (segment (start 150.958824 100) (end 153.3 102.341176) (width 0.2) (layer "F.Cu") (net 4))
 (segment (start 146.5 100) (end 150.958824 100) (width 0.2) (layer "F.Cu") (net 4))
 (segment (start 145.5 96.5) (end 145.5 99) (width 0.2) (layer "F.Cu") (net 4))
 (segment (start 149.88316 111.026) (end 150.199 110.71016) (width 0.2) (layer "F.Cu") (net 10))
 (segment (start 150.199 110.71016) (end 150.199 107.901) (width 0.2) (layer "F.Cu") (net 10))
 (segment (start 144.526 111.026) (end 149.88316 111.026) (width 0.2) (layer "F.Cu") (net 10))
 (segment (start 150.199 107.901) (end 152.1 106) (width 0.2) (layer "F.Cu") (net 10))
 (segment (start 143 109.5) (end 144.526 111.026) (width 0.2) (layer "F.Cu") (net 10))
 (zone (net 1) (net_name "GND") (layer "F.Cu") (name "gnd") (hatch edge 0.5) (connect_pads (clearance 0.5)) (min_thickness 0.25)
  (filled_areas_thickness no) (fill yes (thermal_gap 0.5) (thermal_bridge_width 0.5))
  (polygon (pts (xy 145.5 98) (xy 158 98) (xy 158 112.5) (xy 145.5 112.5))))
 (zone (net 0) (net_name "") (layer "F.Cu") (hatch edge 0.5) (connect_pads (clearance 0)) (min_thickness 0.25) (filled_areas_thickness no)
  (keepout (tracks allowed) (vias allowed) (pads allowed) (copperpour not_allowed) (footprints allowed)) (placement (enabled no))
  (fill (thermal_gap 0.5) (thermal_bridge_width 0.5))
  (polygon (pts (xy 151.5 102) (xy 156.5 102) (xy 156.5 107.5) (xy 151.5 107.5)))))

